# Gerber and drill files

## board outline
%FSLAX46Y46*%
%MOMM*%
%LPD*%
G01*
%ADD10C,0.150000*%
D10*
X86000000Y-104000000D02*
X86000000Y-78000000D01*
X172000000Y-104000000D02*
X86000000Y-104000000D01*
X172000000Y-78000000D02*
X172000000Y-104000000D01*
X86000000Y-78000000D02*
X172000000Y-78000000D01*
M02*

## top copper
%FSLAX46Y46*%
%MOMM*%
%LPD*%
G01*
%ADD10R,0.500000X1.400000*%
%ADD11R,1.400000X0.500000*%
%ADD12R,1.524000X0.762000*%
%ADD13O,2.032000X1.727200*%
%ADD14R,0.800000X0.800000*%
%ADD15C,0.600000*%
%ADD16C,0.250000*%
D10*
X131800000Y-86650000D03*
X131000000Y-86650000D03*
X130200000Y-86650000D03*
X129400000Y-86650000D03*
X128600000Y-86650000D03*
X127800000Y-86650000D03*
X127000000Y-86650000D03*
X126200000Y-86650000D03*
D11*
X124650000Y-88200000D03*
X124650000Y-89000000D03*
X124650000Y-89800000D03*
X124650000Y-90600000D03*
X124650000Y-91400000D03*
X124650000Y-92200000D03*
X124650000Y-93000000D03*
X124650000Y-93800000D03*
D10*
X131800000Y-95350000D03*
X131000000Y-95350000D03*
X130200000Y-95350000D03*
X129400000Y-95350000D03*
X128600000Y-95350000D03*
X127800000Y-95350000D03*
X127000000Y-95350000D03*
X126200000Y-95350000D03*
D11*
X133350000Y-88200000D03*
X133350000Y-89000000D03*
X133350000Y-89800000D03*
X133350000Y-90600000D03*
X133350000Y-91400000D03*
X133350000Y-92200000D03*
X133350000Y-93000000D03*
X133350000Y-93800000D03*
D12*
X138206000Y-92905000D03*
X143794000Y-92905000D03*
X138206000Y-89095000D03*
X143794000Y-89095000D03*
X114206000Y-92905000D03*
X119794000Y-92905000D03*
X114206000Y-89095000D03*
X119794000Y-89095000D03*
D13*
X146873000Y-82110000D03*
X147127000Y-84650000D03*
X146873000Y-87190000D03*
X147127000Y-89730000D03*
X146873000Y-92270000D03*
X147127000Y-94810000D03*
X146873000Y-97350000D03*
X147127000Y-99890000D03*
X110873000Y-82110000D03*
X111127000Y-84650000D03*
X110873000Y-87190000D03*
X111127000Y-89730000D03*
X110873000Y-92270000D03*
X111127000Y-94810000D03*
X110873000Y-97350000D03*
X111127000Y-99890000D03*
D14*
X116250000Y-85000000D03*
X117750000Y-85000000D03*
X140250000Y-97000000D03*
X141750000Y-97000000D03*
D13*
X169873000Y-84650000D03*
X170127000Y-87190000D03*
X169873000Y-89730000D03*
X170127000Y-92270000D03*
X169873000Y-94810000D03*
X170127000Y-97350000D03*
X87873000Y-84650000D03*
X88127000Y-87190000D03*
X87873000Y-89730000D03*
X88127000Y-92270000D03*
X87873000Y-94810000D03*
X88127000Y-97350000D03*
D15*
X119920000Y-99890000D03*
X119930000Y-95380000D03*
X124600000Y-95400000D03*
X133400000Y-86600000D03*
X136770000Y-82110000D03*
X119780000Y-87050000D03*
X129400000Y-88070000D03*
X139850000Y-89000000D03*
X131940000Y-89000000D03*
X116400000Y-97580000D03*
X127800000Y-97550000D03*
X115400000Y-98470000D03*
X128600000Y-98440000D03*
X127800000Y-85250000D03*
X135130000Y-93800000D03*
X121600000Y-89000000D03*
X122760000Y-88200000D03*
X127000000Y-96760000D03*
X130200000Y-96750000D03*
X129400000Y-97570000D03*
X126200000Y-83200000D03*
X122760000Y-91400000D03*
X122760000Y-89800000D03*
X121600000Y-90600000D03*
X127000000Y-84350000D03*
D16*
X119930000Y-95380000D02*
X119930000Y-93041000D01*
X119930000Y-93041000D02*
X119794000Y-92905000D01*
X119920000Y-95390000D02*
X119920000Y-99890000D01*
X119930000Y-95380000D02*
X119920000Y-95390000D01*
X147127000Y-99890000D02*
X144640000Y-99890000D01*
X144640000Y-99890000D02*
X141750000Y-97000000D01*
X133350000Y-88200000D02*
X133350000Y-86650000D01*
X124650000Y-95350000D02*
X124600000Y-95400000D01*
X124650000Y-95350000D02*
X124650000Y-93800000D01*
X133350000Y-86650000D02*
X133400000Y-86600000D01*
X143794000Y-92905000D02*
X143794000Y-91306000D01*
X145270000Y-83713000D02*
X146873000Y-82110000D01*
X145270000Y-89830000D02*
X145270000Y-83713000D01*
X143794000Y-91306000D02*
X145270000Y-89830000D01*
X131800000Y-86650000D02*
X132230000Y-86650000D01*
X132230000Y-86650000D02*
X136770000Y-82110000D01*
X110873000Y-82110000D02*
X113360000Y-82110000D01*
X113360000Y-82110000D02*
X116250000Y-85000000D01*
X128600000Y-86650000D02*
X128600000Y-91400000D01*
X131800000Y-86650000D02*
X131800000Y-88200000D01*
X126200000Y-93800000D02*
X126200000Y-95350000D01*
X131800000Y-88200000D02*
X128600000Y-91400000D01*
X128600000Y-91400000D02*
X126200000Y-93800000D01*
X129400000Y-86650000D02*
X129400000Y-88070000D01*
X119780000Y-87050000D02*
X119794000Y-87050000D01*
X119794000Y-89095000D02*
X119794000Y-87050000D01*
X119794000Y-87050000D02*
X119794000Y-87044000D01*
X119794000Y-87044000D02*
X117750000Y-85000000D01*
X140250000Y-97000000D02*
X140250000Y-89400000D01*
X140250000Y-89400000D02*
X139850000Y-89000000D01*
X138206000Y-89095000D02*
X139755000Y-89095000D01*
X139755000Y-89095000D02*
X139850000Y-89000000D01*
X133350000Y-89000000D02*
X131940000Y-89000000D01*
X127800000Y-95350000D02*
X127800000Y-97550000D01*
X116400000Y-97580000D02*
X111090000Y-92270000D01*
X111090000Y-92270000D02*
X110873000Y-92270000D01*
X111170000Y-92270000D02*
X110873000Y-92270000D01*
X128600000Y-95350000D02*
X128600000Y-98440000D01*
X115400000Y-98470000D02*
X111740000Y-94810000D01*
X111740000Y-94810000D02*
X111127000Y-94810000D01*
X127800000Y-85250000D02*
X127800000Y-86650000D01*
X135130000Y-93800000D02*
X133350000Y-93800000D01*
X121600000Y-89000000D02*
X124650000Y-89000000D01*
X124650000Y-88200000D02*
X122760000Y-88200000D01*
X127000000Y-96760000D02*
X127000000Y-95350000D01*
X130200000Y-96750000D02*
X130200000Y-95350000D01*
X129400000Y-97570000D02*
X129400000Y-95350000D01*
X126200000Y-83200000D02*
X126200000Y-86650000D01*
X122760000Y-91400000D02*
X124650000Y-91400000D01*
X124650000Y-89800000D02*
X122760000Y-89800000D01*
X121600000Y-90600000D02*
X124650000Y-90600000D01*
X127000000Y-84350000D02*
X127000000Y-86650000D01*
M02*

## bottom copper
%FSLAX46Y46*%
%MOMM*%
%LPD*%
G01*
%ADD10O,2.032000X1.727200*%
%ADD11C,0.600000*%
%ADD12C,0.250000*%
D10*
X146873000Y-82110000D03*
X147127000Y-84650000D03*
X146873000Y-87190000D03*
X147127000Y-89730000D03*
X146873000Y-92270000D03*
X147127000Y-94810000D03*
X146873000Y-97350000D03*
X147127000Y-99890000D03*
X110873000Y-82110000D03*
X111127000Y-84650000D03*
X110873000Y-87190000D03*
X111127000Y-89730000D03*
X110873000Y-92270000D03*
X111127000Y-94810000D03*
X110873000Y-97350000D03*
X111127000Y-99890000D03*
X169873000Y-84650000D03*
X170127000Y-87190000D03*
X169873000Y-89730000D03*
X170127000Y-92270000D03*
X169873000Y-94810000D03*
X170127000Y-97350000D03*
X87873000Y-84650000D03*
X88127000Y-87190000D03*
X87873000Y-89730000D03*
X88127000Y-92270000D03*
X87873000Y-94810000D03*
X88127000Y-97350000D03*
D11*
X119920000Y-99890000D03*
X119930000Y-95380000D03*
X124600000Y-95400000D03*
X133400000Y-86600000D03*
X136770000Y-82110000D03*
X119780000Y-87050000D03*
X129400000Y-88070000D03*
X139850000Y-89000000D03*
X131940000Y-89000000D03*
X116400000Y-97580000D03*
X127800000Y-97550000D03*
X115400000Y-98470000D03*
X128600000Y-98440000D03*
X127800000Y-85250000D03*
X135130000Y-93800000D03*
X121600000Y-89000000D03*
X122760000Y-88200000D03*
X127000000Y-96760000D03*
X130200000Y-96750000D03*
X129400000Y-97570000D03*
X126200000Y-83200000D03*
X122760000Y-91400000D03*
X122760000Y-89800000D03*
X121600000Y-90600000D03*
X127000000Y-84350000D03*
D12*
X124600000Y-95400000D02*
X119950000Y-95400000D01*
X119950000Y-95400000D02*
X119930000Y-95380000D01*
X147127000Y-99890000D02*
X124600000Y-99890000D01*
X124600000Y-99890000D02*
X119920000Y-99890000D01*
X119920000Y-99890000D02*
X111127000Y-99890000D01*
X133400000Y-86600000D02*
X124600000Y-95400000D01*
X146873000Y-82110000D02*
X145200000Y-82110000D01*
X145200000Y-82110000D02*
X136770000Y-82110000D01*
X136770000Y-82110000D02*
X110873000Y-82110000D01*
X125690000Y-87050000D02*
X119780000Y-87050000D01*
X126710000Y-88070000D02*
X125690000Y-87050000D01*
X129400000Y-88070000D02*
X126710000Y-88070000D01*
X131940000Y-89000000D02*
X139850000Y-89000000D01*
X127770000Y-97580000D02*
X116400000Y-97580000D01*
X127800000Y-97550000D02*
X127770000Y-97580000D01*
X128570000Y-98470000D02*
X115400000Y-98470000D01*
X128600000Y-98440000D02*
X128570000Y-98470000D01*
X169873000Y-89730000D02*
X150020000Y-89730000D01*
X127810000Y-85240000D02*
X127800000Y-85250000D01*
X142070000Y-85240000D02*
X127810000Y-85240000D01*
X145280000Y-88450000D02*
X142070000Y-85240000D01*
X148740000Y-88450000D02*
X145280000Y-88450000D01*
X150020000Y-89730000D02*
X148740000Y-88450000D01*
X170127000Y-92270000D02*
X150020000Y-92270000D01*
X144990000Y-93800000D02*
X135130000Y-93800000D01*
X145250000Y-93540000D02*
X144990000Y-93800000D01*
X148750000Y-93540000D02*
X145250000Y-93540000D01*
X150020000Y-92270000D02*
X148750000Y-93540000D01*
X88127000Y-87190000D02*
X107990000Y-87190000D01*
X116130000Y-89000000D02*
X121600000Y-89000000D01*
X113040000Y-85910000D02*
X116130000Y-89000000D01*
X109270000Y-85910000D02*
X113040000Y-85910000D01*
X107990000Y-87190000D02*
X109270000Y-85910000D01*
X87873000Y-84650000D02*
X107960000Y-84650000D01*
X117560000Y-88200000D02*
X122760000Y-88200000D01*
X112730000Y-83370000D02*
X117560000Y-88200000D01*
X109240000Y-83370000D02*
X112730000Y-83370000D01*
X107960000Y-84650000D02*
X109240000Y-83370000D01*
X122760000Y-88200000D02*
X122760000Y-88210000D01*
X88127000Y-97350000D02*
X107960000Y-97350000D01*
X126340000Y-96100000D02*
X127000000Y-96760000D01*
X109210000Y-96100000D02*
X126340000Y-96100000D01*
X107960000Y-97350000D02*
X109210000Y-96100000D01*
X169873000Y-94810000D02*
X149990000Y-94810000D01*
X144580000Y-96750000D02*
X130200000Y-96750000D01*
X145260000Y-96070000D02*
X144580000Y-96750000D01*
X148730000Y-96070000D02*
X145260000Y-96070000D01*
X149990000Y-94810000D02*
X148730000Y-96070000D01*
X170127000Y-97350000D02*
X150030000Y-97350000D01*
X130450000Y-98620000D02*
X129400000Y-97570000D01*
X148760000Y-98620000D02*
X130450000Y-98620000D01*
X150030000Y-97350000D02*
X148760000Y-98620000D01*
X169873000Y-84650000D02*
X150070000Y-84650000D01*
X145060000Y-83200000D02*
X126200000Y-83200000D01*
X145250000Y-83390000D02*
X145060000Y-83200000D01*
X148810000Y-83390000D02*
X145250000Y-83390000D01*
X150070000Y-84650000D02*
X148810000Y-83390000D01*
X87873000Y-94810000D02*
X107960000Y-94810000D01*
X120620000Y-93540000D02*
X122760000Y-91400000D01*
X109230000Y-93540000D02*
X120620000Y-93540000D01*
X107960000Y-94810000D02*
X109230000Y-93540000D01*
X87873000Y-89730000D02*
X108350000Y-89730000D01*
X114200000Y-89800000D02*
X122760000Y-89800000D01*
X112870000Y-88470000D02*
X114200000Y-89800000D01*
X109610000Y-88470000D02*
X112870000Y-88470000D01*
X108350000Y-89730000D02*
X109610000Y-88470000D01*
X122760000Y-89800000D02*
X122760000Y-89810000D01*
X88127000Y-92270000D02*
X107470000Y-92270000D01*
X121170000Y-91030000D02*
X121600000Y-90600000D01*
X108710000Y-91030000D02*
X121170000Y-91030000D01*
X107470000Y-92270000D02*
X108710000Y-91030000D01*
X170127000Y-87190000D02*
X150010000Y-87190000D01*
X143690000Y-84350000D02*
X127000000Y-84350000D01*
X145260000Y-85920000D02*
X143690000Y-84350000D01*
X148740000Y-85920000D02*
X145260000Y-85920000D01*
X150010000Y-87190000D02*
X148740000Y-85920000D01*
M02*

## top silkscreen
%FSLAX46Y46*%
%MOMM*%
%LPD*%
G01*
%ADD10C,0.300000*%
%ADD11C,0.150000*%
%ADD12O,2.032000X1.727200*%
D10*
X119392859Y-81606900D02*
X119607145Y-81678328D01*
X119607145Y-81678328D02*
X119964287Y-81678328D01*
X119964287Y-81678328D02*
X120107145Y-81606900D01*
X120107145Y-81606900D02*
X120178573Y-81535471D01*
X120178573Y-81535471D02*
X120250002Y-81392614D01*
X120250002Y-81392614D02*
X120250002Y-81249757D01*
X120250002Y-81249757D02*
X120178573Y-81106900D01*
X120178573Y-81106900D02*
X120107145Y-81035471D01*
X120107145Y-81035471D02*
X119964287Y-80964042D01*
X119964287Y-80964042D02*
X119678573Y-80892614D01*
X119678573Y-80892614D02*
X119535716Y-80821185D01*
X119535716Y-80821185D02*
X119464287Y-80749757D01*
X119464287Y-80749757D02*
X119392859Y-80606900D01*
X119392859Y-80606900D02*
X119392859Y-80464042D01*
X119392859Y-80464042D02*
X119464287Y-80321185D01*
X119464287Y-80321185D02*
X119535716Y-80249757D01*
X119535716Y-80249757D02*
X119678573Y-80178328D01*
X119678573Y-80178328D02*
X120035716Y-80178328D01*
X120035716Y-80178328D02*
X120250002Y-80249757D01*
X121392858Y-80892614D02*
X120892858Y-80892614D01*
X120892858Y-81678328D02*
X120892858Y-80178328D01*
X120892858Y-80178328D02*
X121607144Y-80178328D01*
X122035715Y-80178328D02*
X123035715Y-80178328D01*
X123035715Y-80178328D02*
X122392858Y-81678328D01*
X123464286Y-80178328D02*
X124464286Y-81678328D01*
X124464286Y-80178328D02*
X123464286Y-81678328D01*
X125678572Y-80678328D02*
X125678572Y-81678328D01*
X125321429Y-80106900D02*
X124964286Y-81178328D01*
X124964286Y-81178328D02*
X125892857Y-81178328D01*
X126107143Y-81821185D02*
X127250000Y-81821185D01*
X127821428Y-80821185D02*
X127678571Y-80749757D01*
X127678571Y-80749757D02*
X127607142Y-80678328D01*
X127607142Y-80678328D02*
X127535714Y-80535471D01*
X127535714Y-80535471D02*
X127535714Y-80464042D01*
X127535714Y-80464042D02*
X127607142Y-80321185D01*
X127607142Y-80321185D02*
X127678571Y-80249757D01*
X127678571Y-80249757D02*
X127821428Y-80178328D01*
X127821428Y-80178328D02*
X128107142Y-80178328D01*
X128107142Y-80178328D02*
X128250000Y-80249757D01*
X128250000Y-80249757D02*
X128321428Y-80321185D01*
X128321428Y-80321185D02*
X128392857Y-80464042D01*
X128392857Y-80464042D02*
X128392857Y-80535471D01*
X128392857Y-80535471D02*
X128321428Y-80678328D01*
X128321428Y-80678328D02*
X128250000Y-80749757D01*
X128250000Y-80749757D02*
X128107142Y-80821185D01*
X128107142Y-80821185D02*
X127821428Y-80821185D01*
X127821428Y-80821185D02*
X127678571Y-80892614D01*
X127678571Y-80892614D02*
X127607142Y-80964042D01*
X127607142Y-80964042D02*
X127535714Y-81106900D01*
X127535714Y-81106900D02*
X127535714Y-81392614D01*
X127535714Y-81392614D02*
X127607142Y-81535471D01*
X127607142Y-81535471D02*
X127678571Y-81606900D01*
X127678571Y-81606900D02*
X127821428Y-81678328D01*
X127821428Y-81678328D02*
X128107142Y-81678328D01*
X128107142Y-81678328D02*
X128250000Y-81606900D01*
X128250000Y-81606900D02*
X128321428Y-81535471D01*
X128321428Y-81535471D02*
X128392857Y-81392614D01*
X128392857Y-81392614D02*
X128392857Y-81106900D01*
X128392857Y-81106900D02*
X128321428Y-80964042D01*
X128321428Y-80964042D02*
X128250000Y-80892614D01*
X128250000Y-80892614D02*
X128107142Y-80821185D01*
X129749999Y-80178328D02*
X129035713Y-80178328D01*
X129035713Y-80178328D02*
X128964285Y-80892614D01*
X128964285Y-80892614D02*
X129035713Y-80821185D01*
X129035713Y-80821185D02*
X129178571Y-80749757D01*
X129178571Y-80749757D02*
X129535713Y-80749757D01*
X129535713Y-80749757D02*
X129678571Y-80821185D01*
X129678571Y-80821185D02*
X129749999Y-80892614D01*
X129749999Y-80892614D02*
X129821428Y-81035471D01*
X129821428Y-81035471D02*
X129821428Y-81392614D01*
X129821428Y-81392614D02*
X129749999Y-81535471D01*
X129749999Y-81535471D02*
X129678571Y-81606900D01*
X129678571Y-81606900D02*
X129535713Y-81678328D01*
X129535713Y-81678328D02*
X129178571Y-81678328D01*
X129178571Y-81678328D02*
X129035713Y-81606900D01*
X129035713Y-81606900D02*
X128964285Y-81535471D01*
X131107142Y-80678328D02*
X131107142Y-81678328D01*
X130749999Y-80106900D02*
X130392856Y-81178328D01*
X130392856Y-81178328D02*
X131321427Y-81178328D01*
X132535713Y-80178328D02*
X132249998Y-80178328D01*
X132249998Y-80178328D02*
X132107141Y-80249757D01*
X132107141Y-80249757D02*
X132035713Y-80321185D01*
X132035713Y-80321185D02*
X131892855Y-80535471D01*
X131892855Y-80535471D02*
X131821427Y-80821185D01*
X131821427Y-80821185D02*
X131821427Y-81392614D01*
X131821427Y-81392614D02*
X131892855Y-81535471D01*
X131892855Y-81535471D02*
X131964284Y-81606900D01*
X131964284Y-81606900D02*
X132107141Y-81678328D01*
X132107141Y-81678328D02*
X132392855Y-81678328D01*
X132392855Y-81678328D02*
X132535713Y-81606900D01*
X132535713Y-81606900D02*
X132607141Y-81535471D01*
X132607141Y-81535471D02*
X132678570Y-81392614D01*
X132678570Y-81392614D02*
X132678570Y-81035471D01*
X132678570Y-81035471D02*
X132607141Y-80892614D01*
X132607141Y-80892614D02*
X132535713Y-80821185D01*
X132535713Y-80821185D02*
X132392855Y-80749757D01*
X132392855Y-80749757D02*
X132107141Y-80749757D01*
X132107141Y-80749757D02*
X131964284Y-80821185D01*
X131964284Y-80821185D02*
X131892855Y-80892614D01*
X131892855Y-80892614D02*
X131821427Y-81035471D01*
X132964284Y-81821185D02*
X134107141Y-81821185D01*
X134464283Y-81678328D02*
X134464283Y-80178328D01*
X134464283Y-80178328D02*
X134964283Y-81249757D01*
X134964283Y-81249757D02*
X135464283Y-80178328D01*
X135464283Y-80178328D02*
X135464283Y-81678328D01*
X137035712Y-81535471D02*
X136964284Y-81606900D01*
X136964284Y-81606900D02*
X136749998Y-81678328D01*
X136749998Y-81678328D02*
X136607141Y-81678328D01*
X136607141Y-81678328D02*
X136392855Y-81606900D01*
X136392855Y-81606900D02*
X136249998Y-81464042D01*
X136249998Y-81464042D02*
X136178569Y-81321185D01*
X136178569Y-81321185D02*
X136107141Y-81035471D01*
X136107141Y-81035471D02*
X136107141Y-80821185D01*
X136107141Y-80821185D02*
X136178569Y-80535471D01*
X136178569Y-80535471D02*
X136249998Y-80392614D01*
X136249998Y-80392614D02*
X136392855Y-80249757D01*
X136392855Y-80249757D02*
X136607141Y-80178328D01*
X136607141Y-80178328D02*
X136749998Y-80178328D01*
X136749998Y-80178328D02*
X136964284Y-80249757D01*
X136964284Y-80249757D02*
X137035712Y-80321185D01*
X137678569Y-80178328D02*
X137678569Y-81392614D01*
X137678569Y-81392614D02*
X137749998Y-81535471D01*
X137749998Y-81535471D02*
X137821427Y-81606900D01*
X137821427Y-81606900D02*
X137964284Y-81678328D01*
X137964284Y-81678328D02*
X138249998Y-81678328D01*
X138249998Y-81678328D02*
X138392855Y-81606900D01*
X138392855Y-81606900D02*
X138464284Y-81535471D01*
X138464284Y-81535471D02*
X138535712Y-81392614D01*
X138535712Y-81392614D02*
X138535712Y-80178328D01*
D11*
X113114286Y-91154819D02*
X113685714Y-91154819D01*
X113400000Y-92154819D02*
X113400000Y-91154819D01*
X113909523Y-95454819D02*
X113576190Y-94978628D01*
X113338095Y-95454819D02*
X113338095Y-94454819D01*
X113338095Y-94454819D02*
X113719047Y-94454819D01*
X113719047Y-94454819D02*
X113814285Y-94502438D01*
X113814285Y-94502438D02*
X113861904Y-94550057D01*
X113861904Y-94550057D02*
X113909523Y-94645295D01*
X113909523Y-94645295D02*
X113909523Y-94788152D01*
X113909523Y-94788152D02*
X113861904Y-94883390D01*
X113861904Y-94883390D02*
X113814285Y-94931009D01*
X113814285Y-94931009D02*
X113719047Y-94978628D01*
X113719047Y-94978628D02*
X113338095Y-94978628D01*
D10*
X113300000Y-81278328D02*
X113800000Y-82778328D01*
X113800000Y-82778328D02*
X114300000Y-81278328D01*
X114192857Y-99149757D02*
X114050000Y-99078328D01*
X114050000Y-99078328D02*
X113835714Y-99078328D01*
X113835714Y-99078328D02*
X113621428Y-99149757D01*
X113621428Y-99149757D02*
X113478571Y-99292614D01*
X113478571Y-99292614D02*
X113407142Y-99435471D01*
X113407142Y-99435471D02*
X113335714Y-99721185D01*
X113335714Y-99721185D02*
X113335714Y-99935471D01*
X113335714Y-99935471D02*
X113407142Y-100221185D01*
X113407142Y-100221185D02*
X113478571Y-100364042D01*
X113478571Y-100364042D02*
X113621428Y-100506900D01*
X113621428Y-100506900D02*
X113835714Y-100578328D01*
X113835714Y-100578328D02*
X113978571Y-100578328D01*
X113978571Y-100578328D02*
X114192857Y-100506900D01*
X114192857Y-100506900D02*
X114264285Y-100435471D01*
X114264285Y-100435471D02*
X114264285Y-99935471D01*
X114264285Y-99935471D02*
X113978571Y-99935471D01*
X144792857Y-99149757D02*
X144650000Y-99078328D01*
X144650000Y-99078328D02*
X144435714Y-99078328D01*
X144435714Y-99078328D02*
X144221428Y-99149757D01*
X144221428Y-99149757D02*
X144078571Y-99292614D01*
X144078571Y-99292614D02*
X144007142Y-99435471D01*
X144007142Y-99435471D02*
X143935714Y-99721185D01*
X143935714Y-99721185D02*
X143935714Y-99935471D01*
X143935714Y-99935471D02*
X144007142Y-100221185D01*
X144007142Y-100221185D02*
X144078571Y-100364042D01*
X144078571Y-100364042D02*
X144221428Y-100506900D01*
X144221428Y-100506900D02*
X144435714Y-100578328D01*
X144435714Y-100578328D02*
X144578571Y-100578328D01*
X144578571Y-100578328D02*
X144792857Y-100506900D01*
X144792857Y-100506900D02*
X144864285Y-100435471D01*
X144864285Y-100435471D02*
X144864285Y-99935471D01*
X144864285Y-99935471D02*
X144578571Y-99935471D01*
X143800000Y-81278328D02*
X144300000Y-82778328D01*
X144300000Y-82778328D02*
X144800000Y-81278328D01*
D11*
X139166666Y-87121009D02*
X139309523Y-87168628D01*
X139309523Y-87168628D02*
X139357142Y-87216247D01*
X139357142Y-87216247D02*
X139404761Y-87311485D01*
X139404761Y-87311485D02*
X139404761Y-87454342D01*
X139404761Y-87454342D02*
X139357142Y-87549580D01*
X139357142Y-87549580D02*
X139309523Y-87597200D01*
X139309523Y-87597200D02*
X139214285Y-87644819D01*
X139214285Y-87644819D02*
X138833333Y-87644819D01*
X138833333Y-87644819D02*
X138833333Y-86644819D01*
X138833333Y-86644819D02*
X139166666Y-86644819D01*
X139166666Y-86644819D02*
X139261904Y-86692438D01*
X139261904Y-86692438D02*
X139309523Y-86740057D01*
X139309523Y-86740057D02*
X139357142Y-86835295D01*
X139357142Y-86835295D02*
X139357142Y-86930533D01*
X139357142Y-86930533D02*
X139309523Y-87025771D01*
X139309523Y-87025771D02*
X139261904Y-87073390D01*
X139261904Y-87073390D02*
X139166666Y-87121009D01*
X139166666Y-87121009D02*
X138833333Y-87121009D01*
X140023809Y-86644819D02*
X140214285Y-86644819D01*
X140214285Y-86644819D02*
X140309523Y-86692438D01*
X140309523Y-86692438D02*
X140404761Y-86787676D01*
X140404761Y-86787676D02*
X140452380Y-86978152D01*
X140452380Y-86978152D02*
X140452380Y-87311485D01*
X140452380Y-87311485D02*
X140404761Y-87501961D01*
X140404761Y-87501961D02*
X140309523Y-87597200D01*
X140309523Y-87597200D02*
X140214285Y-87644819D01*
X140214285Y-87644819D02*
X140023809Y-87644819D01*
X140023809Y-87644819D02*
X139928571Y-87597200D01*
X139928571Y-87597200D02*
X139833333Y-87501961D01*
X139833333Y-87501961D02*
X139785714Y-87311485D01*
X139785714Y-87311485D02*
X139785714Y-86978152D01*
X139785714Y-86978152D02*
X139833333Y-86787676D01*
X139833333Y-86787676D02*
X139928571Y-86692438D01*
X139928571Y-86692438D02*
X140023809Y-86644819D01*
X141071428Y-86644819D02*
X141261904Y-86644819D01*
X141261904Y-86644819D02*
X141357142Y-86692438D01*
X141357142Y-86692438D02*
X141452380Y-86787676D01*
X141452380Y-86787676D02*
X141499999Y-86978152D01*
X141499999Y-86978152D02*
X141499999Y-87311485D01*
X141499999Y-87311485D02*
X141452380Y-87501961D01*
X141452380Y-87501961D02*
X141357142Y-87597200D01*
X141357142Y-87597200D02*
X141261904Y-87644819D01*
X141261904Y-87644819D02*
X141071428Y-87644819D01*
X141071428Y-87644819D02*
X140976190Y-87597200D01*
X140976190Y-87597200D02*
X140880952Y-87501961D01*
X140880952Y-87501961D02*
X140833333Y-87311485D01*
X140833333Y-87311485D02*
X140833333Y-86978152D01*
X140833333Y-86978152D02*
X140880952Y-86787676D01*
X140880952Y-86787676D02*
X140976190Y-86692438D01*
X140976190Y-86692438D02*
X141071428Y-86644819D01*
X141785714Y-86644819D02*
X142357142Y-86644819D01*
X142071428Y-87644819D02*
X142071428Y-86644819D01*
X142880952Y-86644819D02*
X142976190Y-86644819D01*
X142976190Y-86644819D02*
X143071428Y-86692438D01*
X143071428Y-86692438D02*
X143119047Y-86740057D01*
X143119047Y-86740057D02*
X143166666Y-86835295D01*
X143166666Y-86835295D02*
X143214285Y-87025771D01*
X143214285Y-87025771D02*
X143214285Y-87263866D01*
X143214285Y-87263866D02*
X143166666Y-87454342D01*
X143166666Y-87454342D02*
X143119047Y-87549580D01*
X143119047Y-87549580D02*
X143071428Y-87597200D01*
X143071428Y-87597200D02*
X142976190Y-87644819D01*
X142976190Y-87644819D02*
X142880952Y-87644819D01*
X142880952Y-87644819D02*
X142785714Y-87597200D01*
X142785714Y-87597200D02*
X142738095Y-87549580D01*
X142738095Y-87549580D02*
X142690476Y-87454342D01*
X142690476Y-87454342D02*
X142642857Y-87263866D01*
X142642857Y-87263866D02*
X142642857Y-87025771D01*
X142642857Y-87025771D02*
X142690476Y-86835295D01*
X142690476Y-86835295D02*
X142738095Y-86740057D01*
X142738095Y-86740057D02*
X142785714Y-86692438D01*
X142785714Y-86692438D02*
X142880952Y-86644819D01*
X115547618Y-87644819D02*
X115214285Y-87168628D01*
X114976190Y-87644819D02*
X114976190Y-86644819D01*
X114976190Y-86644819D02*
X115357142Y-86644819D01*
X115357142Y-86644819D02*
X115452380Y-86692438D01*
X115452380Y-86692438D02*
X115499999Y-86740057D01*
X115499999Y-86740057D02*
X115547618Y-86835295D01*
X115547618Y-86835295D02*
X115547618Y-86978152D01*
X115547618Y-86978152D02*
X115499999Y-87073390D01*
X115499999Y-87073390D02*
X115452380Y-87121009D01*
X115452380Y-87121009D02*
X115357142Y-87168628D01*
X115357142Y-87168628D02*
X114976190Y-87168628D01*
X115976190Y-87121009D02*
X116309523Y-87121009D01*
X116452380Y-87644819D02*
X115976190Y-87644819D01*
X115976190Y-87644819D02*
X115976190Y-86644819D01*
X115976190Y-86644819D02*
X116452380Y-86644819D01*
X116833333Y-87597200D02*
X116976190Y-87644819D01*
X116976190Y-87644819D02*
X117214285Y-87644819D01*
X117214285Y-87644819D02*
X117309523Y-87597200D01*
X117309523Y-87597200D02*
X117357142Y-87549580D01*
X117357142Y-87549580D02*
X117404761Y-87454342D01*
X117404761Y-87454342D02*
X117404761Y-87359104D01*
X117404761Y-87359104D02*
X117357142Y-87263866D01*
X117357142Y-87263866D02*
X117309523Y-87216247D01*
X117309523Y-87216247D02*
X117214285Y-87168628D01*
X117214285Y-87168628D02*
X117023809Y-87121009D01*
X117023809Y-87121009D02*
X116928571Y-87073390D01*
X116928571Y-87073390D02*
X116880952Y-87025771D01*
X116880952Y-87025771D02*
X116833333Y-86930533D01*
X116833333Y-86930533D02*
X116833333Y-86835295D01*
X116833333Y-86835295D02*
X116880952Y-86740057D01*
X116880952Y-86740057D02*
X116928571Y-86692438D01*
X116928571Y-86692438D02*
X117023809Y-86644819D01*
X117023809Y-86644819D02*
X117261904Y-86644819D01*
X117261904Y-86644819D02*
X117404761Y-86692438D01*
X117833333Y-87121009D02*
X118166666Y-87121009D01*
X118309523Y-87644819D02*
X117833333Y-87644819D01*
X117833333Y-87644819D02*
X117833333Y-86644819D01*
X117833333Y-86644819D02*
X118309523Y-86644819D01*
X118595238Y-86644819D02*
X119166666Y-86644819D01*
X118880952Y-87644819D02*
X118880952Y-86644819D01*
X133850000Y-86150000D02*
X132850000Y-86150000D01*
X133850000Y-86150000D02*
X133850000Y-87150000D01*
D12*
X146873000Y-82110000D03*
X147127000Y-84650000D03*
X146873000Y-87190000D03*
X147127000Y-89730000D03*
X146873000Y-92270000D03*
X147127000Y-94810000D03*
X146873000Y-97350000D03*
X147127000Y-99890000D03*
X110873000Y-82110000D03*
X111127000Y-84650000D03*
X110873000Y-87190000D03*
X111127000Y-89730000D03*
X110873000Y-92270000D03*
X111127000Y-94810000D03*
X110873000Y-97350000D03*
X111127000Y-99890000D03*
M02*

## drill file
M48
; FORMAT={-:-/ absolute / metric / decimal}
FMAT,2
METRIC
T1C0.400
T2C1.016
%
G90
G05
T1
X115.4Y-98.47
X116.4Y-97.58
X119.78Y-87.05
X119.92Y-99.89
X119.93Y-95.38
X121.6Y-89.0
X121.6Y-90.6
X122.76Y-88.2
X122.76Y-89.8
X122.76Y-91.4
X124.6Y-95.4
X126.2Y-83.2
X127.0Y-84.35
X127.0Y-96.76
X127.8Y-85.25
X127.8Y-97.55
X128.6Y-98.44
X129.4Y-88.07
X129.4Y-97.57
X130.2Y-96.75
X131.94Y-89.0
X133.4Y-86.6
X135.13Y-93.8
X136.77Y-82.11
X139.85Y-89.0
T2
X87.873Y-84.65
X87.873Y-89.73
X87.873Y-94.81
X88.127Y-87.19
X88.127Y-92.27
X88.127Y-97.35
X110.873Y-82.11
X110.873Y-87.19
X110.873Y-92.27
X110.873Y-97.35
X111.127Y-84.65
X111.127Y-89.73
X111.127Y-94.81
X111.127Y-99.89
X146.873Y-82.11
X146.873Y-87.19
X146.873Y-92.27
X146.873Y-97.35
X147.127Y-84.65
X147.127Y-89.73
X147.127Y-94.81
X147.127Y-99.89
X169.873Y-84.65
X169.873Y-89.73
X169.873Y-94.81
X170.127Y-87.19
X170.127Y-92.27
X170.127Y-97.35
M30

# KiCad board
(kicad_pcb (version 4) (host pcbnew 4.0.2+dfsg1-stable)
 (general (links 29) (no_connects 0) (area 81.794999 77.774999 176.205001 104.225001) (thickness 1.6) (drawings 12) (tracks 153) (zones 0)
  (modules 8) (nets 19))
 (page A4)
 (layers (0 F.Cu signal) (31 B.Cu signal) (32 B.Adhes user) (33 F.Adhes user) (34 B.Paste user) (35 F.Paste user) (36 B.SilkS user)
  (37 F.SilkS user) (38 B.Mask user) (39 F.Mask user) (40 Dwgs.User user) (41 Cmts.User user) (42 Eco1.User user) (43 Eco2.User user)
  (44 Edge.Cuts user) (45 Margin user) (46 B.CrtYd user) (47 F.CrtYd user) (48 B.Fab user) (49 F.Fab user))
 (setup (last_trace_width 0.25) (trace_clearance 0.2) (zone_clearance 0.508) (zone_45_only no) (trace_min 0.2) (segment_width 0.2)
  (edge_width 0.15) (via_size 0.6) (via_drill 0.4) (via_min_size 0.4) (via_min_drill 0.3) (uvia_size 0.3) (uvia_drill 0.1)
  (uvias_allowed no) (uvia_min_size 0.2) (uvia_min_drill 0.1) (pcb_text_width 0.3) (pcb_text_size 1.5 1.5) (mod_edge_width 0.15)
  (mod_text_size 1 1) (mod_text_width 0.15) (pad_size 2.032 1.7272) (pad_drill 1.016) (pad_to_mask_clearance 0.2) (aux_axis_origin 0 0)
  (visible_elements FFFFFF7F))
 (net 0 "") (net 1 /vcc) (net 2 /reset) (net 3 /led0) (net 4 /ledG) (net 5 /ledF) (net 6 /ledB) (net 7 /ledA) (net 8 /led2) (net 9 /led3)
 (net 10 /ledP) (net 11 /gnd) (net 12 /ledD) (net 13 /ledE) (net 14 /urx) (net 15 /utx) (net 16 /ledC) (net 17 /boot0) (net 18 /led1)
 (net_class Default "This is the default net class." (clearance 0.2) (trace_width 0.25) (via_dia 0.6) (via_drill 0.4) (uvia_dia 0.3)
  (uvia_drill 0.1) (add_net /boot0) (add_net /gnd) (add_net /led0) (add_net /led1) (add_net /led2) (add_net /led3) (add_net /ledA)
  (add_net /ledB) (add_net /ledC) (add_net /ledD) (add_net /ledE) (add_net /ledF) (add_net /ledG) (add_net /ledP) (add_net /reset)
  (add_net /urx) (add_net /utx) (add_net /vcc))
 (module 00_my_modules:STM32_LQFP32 (layer F.Cu) (at 129 91 270)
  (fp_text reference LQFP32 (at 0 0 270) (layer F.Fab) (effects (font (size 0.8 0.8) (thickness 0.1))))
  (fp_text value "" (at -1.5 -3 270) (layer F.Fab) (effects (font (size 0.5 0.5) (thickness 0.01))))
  (fp_line (start -4.85 -4.85) (end -4.85 -3.85) (layer F.SilkS) (width 0.15))
  (fp_line (start -4.85 -4.85) (end -3.85 -4.85) (layer F.SilkS) (width 0.15))
  (pad 3.3 smd rect (at -4.35 -2.8 270) (size 1.4 0.5) (layers F.Cu F.Paste F.Mask) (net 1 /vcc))
  (pad PF0 smd rect (at -4.35 -2 270) (size 1.4 0.5) (layers F.Cu F.Paste F.Mask))
  (pad PF1 smd rect (at -4.35 -1.2 270) (size 1.4 0.5) (layers F.Cu F.Paste F.Mask))
  (pad RST smd rect (at -4.35 -0.4 270) (size 1.4 0.5) (layers F.Cu F.Paste F.Mask) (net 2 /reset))
  (pad 3.3 smd rect (at -4.35 0.4 270) (size 1.4 0.5) (layers F.Cu F.Paste F.Mask) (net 1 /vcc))
  (pad PA0 smd rect (at -4.35 1.2 270) (size 1.4 0.5) (layers F.Cu F.Paste F.Mask) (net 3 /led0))
  (pad PA1 smd rect (at -4.35 2 270) (size 1.4 0.5) (layers F.Cu F.Paste F.Mask) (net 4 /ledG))
  (pad PA2 smd rect (at -4.35 2.8 270) (size 1.4 0.5) (layers F.Cu F.Paste F.Mask) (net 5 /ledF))
  (pad PA3 smd rect (at -2.8 4.35) (size 1.4 0.5) (layers F.Cu F.Paste F.Mask) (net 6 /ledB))
  (pad PA4 smd rect (at -2 4.35) (size 1.4 0.5) (layers F.Cu F.Paste F.Mask) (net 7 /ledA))
  (pad PA5 smd rect (at -1.2 4.35) (size 1.4 0.5) (layers F.Cu F.Paste F.Mask) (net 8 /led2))
  (pad PA6 smd rect (at -0.4 4.35) (size 1.4 0.5) (layers F.Cu F.Paste F.Mask) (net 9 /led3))
  (pad PA7 smd rect (at 0.4 4.35) (size 1.4 0.5) (layers F.Cu F.Paste F.Mask) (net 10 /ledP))
  (pad PB0 smd rect (at 1.2 4.35) (size 1.4 0.5) (layers F.Cu F.Paste F.Mask))
  (pad PB1 smd rect (at 2 4.35) (size 1.4 0.5) (layers F.Cu F.Paste F.Mask))
  (pad GND smd rect (at 2.8 4.35) (size 1.4 0.5) (layers F.Cu F.Paste F.Mask) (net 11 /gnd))
  (pad PA14 smd rect (at 4.35 -2.8 270) (size 1.4 0.5) (layers F.Cu F.Paste F.Mask))
  (pad PA13 smd rect (at 4.35 -2 270) (size 1.4 0.5) (layers F.Cu F.Paste F.Mask))
  (pad PA12 smd rect (at 4.35 -1.2 270) (size 1.4 0.5) (layers F.Cu F.Paste F.Mask) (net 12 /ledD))
  (pad PA11 smd rect (at 4.35 -0.4 270) (size 1.4 0.5) (layers F.Cu F.Paste F.Mask) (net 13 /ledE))
  (pad PA10 smd rect (at 4.35 0.4 270) (size 1.4 0.5) (layers F.Cu F.Paste F.Mask) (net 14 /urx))
  (pad PA9 smd rect (at 4.35 1.2 270) (size 1.4 0.5) (layers F.Cu F.Paste F.Mask) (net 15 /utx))
  (pad PA8 smd rect (at 4.35 2 270) (size 1.4 0.5) (layers F.Cu F.Paste F.Mask) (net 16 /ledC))
  (pad 3.3 smd rect (at 4.35 2.8 270) (size 1.4 0.5) (layers F.Cu F.Paste F.Mask) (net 1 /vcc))
  (pad GND smd rect (at -2.8 -4.35) (size 1.4 0.5) (layers F.Cu F.Paste F.Mask) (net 11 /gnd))
  (pad BOOT smd rect (at -2 -4.35) (size 1.4 0.5) (layers F.Cu F.Paste F.Mask) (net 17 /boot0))
  (pad PB7 smd rect (at -1.2 -4.35) (size 1.4 0.5) (layers F.Cu F.Paste F.Mask))
  (pad PB6 smd rect (at -0.4 -4.35) (size 1.4 0.5) (layers F.Cu F.Paste F.Mask))
  (pad PB5 smd rect (at 0.4 -4.35) (size 1.4 0.5) (layers F.Cu F.Paste F.Mask))
  (pad PB4 smd rect (at 1.2 -4.35) (size 1.4 0.5) (layers F.Cu F.Paste F.Mask))
  (pad PB3 smd rect (at 2 -4.35) (size 1.4 0.5) (layers F.Cu F.Paste F.Mask))
  (pad PA15 smd rect (at 2.8 -4.35) (size 1.4 0.5) (layers F.Cu F.Paste F.Mask) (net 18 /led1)))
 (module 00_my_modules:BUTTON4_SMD (layer F.Cu) (at 141 91)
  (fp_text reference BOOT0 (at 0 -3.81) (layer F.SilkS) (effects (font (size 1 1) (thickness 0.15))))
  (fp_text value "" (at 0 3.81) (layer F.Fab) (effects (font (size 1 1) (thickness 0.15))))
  (pad 1 smd rect (at -2.794 1.905) (size 1.524 0.762) (layers F.Cu F.Paste F.Mask))
  (pad 2 smd rect (at 2.794 1.905) (size 1.524 0.762) (layers F.Cu F.Paste F.Mask) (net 1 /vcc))
  (pad 3 smd rect (at -2.794 -1.905) (size 1.524 0.762) (layers F.Cu F.Paste F.Mask) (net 17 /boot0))
  (pad 4 smd rect (at 2.794 -1.905) (size 1.524 0.762) (layers F.Cu F.Paste F.Mask)))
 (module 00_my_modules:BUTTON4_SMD (layer F.Cu) (at 117 91)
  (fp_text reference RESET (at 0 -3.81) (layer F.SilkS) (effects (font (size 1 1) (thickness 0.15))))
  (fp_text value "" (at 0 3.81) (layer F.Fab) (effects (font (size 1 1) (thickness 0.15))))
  (pad 1 smd rect (at -2.794 1.905) (size 1.524 0.762) (layers F.Cu F.Paste F.Mask))
  (pad 2 smd rect (at 2.794 1.905) (size 1.524 0.762) (layers F.Cu F.Paste F.Mask) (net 11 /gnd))
  (pad 3 smd rect (at -2.794 -1.905) (size 1.524 0.762) (layers F.Cu F.Paste F.Mask))
  (pad 4 smd rect (at 2.794 -1.905) (size 1.524 0.762) (layers F.Cu F.Paste F.Mask) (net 2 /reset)))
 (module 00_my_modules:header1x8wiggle (layer F.Cu) (at 147 91)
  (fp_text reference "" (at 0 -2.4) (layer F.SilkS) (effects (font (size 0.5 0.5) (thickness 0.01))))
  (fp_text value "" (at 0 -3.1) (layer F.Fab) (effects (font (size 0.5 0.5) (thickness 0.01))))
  (pad 1 thru_hole oval (at -0.127 -8.89) (size 2.032 1.7272) (drill 1.016) (layers *.Cu *.Mask F.SilkS) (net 1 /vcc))
  (pad 2 thru_hole oval (at 0.127 -6.35) (size 2.032 1.7272) (drill 1.016) (layers *.Cu *.Mask F.SilkS))
  (pad 3 thru_hole oval (at -0.127 -3.81) (size 2.032 1.7272) (drill 1.016) (layers *.Cu *.Mask F.SilkS))
  (pad 4 thru_hole oval (at 0.127 -1.27) (size 2.032 1.7272) (drill 1.016) (layers *.Cu *.Mask F.SilkS))
  (pad 5 thru_hole oval (at -0.127 1.27) (size 2.032 1.7272) (drill 1.016) (layers *.Cu *.Mask F.SilkS))
  (pad 6 thru_hole oval (at 0.127 3.81) (size 2.032 1.7272) (drill 1.016) (layers *.Cu *.Mask F.SilkS))
  (pad 7 thru_hole oval (at -0.127 6.35) (size 2.032 1.7272) (drill 1.016) (layers *.Cu *.Mask F.SilkS))
  (pad 8 thru_hole oval (at 0.127 8.89) (size 2.032 1.7272) (drill 1.016) (layers *.Cu *.Mask F.SilkS) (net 11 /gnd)))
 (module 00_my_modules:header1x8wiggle (layer F.Cu) (at 111 91)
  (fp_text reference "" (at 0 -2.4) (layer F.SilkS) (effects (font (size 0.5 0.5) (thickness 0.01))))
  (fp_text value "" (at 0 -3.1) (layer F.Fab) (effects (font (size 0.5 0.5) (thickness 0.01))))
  (pad 1 thru_hole oval (at -0.127 -8.89) (size 2.032 1.7272) (drill 1.016) (layers *.Cu *.Mask F.SilkS) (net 1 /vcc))
  (pad 2 thru_hole oval (at 0.127 -6.35) (size 2.032 1.7272) (drill 1.016) (layers *.Cu *.Mask F.SilkS))
  (pad 3 thru_hole oval (at -0.127 -3.81) (size 2.032 1.7272) (drill 1.016) (layers *.Cu *.Mask F.SilkS))
  (pad 4 thru_hole oval (at 0.127 -1.27) (size 2.032 1.7272) (drill 1.016) (layers *.Cu *.Mask F.SilkS))
  (pad 5 thru_hole oval (at -0.127 1.27) (size 2.032 1.7272) (drill 1.016) (layers *.Cu *.Mask F.SilkS) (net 15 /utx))
  (pad 6 thru_hole oval (at 0.127 3.81) (size 2.032 1.7272) (drill 1.016) (layers *.Cu *.Mask F.SilkS) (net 14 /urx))
  (pad 7 thru_hole oval (at -0.127 6.35) (size 2.032 1.7272) (drill 1.016) (layers *.Cu *.Mask F.SilkS))
  (pad 8 thru_hole oval (at 0.127 8.89) (size 2.032 1.7272) (drill 1.016) (layers *.Cu *.Mask F.SilkS) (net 11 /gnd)))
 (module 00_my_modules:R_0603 (layer F.Cu) (at 117 85)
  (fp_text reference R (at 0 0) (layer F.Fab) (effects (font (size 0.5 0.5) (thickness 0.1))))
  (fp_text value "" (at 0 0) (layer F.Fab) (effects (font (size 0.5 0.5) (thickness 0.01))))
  (pad 1 smd rect (at -0.75 0) (size 0.8 0.8) (layers F.Cu F.Paste F.Mask) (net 1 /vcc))
  (pad 2 smd rect (at 0.75 0) (size 0.8 0.8) (layers F.Cu F.Paste F.Mask) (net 2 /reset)))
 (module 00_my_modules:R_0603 (layer F.Cu) (at 141 97)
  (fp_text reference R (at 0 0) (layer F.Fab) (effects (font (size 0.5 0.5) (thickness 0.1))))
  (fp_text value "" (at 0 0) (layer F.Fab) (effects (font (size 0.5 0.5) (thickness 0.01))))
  (pad 1 smd rect (at -0.75 0) (size 0.8 0.8) (layers F.Cu F.Paste F.Mask) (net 17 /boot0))
  (pad 2 smd rect (at 0.75 0) (size 0.8 0.8) (layers F.Cu F.Paste F.Mask) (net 11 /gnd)))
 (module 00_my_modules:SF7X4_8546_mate (layer B.Cu) (at 129 91 180)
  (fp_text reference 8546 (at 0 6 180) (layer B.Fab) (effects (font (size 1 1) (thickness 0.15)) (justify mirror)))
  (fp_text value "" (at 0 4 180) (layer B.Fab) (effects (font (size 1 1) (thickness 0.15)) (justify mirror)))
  (pad F thru_hole oval (at -40.873 6.35 180) (size 2.032 1.7272) (drill 1.016) (layers *.Cu *.Mask B.SilkS) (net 5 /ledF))
  (pad G thru_hole oval (at -41.127 3.81 180) (size 2.032 1.7272) (drill 1.016) (layers *.Cu *.Mask B.SilkS) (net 4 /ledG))
  (pad V0 thru_hole oval (at -40.873 1.27 180) (size 2.032 1.7272) (drill 1.016) (layers *.Cu *.Mask B.SilkS) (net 3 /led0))
  (pad V1 thru_hole oval (at -41.127 -1.27 180) (size 2.032 1.7272) (drill 1.016) (layers *.Cu *.Mask B.SilkS) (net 18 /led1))
  (pad D thru_hole oval (at -40.873 -3.81 180) (size 2.032 1.7272) (drill 1.016) (layers *.Cu *.Mask B.SilkS) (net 12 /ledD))
  (pad E thru_hole oval (at -41.127 -6.35 180) (size 2.032 1.7272) (drill 1.016) (layers *.Cu *.Mask B.SilkS) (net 13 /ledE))
  (pad B thru_hole oval (at 41.127 6.35 180) (size 2.032 1.7272) (drill 1.016) (layers *.Cu *.Mask B.SilkS) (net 6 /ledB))
  (pad A thru_hole oval (at 40.873 3.81 180) (size 2.032 1.7272) (drill 1.016) (layers *.Cu *.Mask B.SilkS) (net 7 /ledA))
  (pad V2 thru_hole oval (at 41.127 1.27 180) (size 2.032 1.7272) (drill 1.016) (layers *.Cu *.Mask B.SilkS) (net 8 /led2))
  (pad V3 thru_hole oval (at 40.873 -1.27 180) (size 2.032 1.7272) (drill 1.016) (layers *.Cu *.Mask B.SilkS) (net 9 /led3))
  (pad P thru_hole oval (at 41.127 -3.81 180) (size 2.032 1.7272) (drill 1.016) (layers *.Cu *.Mask B.SilkS) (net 10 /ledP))
  (pad C thru_hole oval (at 40.873 -6.35 180) (size 2.032 1.7272) (drill 1.016) (layers *.Cu *.Mask B.SilkS) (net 16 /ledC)))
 (gr_line (start 86 104) (end 86 78) (angle 90) (layer Edge.Cuts) (width 0.15))
 (gr_line (start 172 104) (end 86 104) (angle 90) (layer Edge.Cuts) (width 0.15))
 (gr_line (start 172 78) (end 172 104) (angle 90) (layer Edge.Cuts) (width 0.15))
 (gr_line (start 86 78) (end 172 78) (angle 90) (layer Edge.Cuts) (width 0.15))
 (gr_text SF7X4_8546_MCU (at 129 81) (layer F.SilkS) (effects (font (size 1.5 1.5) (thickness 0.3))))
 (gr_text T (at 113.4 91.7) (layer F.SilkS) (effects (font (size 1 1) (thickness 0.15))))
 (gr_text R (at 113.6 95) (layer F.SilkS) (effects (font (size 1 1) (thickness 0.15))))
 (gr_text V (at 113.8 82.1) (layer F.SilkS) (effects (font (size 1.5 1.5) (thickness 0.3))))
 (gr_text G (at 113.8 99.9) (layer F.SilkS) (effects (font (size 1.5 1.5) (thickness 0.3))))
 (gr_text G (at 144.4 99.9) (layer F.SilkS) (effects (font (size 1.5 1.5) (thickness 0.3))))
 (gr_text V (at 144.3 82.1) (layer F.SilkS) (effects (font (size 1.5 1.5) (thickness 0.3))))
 (segment (start 119.93 95.38) (end 119.93 93.041) (width 0.25) (layer F.Cu) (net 11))
 (segment (start 119.93 93.041) (end 119.794 92.905) (width 0.25) (layer F.Cu) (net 11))
 (segment (start 124.6 95.4) (end 119.95 95.4) (width 0.25) (layer B.Cu) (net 11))
 (via (at 119.92 99.89) (size 0.6) (drill 0.4) (layers F.Cu B.Cu) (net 11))
 (segment (start 119.92 95.39) (end 119.92 99.89) (width 0.25) (layer F.Cu) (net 11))
 (segment (start 119.93 95.38) (end 119.92 95.39) (width 0.25) (layer F.Cu) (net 11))
 (via (at 119.93 95.38) (size 0.6) (drill 0.4) (layers F.Cu B.Cu) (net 11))
 (segment (start 119.95 95.4) (end 119.93 95.38) (width 0.25) (layer B.Cu) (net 11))
 (segment (start 147.127 99.89) (end 144.64 99.89) (width 0.25) (layer F.Cu) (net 11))
 (segment (start 144.64 99.89) (end 141.75 97) (width 0.25) (layer F.Cu) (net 11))
 (segment (start 147.127 99.89) (end 124.6 99.89) (width 0.25) (layer B.Cu) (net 11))
 (segment (start 124.6 99.89) (end 119.92 99.89) (width 0.25) (layer B.Cu) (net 11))
 (segment (start 119.92 99.89) (end 111.127 99.89) (width 0.25) (layer B.Cu) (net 11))
 (segment (start 133.35 88.2) (end 133.35 86.65) (width 0.25) (layer F.Cu) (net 11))
 (segment (start 124.65 95.35) (end 124.6 95.4) (width 0.25) (layer F.Cu) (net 11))
 (via (at 124.6 95.4) (size 0.6) (drill 0.4) (layers F.Cu B.Cu) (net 11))
 (segment (start 124.65 95.35) (end 124.65 93.8) (width 0.25) (layer F.Cu) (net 11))
 (segment (start 133.4 86.6) (end 124.6 95.4) (width 0.25) (layer B.Cu) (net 11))
 (via (at 133.4 86.6) (size 0.6) (drill 0.4) (layers F.Cu B.Cu) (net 11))
 (segment (start 133.35 86.65) (end 133.4 86.6) (width 0.25) (layer F.Cu) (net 11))
 (segment (start 143.794 92.905) (end 143.794 91.306) (width 0.25) (layer F.Cu) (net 1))
 (segment (start 145.27 83.713) (end 146.873 82.11) (width 0.25) (layer F.Cu) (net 1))
 (segment (start 145.27 89.83) (end 145.27 83.713) (width 0.25) (layer F.Cu) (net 1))
 (segment (start 143.794 91.306) (end 145.27 89.83) (width 0.25) (layer F.Cu) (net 1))
 (segment (start 131.8 86.65) (end 132.23 86.65) (width 0.25) (layer F.Cu) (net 1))
 (via (at 136.77 82.11) (size 0.6) (drill 0.4) (layers F.Cu B.Cu) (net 1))
 (segment (start 132.23 86.65) (end 136.77 82.11) (width 0.25) (layer F.Cu) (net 1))
 (segment (start 110.873 82.11) (end 113.36 82.11) (width 0.25) (layer F.Cu) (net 1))
 (segment (start 113.36 82.11) (end 116.25 85) (width 0.25) (layer F.Cu) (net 1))
 (segment (start 146.873 82.11) (end 145.2 82.11) (width 0.25) (layer B.Cu) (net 1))
 (segment (start 145.2 82.11) (end 136.77 82.11) (width 0.25) (layer B.Cu) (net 1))
 (segment (start 136.77 82.11) (end 110.873 82.11) (width 0.25) (layer B.Cu) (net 1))
 (segment (start 128.6 86.65) (end 128.6 91.4) (width 0.25) (layer F.Cu) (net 1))
 (segment (start 131.8 86.65) (end 131.8 88.2) (width 0.25) (layer F.Cu) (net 1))
 (segment (start 126.2 93.8) (end 126.2 95.35) (width 0.25) (layer F.Cu) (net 1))
 (segment (start 131.8 88.2) (end 128.6 91.4) (width 0.25) (layer F.Cu) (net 1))
 (segment (start 128.6 91.4) (end 126.2 93.8) (width 0.25) (layer F.Cu) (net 1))
 (segment (start 129.4 86.65) (end 129.4 88.07) (width 0.25) (layer F.Cu) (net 2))
 (segment (start 119.78 87.05) (end 119.794 87.05) (width 0.25) (layer F.Cu) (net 2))
 (via (at 119.78 87.05) (size 0.6) (drill 0.4) (layers F.Cu B.Cu) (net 2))
 (segment (start 125.69 87.05) (end 119.78 87.05) (width 0.25) (layer B.Cu) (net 2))
 (segment (start 126.71 88.07) (end 125.69 87.05) (width 0.25) (layer B.Cu) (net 2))
 (segment (start 129.4 88.07) (end 126.71 88.07) (width 0.25) (layer B.Cu) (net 2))
 (via (at 129.4 88.07) (size 0.6) (drill 0.4) (layers F.Cu B.Cu) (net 2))
 (segment (start 119.794 89.095) (end 119.794 87.05) (width 0.25) (layer F.Cu) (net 2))
 (segment (start 119.794 87.05) (end 119.794 87.044) (width 0.25) (layer F.Cu) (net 2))
 (segment (start 119.794 87.044) (end 117.75 85) (width 0.25) (layer F.Cu) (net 2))
 (segment (start 140.25 97) (end 140.25 89.4) (width 0.25) (layer F.Cu) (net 17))
 (segment (start 140.25 89.4) (end 139.85 89) (width 0.25) (layer F.Cu) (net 17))
 (via (at 139.85 89) (size 0.6) (drill 0.4) (layers F.Cu B.Cu) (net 17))
 (segment (start 138.206 89.095) (end 139.755 89.095) (width 0.25) (layer F.Cu) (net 17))
 (segment (start 139.755 89.095) (end 139.85 89) (width 0.25) (layer F.Cu) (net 17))
 (segment (start 133.35 89) (end 131.94 89) (width 0.25) (layer F.Cu) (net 17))
 (segment (start 131.94 89) (end 139.85 89) (width 0.25) (layer B.Cu) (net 17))
 (via (at 131.94 89) (size 0.6) (drill 0.4) (layers F.Cu B.Cu) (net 17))
 (segment (start 127.8 95.35) (end 127.8 97.55) (width 0.25) (layer F.Cu) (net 15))
 (segment (start 116.4 97.58) (end 111.09 92.27) (width 0.25) (layer F.Cu) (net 15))
 (via (at 116.4 97.58) (size 0.6) (drill 0.4) (layers F.Cu B.Cu) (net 15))
 (segment (start 127.77 97.58) (end 116.4 97.58) (width 0.25) (layer B.Cu) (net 15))
 (segment (start 127.8 97.55) (end 127.77 97.58) (width 0.25) (layer B.Cu) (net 15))
 (via (at 127.8 97.55) (size 0.6) (drill 0.4) (layers F.Cu B.Cu) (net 15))
 (segment (start 111.09 92.27) (end 110.873 92.27) (width 0.25) (layer F.Cu) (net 15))
 (segment (start 111.17 92.27) (end 110.873 92.27) (width 0.25) (layer F.Cu) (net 15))
 (segment (start 128.6 95.35) (end 128.6 98.44) (width 0.25) (layer F.Cu) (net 14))
 (segment (start 115.4 98.47) (end 111.74 94.81) (width 0.25) (layer F.Cu) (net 14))
 (via (at 115.4 98.47) (size 0.6) (drill 0.4) (layers F.Cu B.Cu) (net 14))
 (segment (start 128.57 98.47) (end 115.4 98.47) (width 0.25) (layer B.Cu) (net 14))
 (segment (start 128.6 98.44) (end 128.57 98.47) (width 0.25) (layer B.Cu) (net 14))
 (via (at 128.6 98.44) (size 0.6) (drill 0.4) (layers F.Cu B.Cu) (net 14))
 (segment (start 111.74 94.81) (end 111.127 94.81) (width 0.25) (layer F.Cu) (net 14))
 (segment (start 169.873 89.73) (end 150.02 89.73) (width 0.25) (layer B.Cu) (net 3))
 (via (at 127.8 85.25) (size 0.6) (drill 0.4) (layers F.Cu B.Cu) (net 3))
 (segment (start 127.8 85.25) (end 127.8 86.65) (width 0.25) (layer F.Cu) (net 3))
 (segment (start 127.81 85.24) (end 127.8 85.25) (width 0.25) (layer B.Cu) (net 3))
 (segment (start 142.07 85.24) (end 127.81 85.24) (width 0.25) (layer B.Cu) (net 3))
 (segment (start 145.28 88.45) (end 142.07 85.24) (width 0.25) (layer B.Cu) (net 3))
 (segment (start 148.74 88.45) (end 145.28 88.45) (width 0.25) (layer B.Cu) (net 3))
 (segment (start 150.02 89.73) (end 148.74 88.45) (width 0.25) (layer B.Cu) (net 3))
 (segment (start 170.127 92.27) (end 150.02 92.27) (width 0.25) (layer B.Cu) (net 18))
 (via (at 135.13 93.8) (size 0.6) (drill 0.4) (layers F.Cu B.Cu) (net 18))
 (segment (start 135.13 93.8) (end 133.35 93.8) (width 0.25) (layer F.Cu) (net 18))
 (segment (start 144.99 93.8) (end 135.13 93.8) (width 0.25) (layer B.Cu) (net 18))
 (segment (start 145.25 93.54) (end 144.99 93.8) (width 0.25) (layer B.Cu) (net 18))
 (segment (start 148.75 93.54) (end 145.25 93.54) (width 0.25) (layer B.Cu) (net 18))
 (segment (start 150.02 92.27) (end 148.75 93.54) (width 0.25) (layer B.Cu) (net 18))
 (segment (start 88.127 87.19) (end 107.99 87.19) (width 0.25) (layer B.Cu) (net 7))
 (via (at 121.6 89) (size 0.6) (drill 0.4) (layers F.Cu B.Cu) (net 7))
 (segment (start 121.6 89) (end 124.65 89) (width 0.25) (layer F.Cu) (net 7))
 (segment (start 116.13 89) (end 121.6 89) (width 0.25) (layer B.Cu) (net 7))
 (segment (start 113.04 85.91) (end 116.13 89) (width 0.25) (layer B.Cu) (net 7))
 (segment (start 109.27 85.91) (end 113.04 85.91) (width 0.25) (layer B.Cu) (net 7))
 (segment (start 107.99 87.19) (end 109.27 85.91) (width 0.25) (layer B.Cu) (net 7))
 (segment (start 87.873 84.65) (end 107.96 84.65) (width 0.25) (layer B.Cu) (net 6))
 (segment (start 117.56 88.2) (end 122.76 88.2) (width 0.25) (layer B.Cu) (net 6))
 (segment (start 112.73 83.37) (end 117.56 88.2) (width 0.25) (layer B.Cu) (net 6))
 (segment (start 109.24 83.37) (end 112.73 83.37) (width 0.25) (layer B.Cu) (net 6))
 (segment (start 107.96 84.65) (end 109.24 83.37) (width 0.25) (layer B.Cu) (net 6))
 (segment (start 124.65 88.2) (end 122.76 88.2) (width 0.25) (layer F.Cu) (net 6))
 (segment (start 122.76 88.2) (end 122.76 88.21) (width 0.25) (layer B.Cu) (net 6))
 (via (at 122.76 88.2) (size 0.6) (drill 0.4) (layers F.Cu B.Cu) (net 6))
 (segment (start 88.127 97.35) (end 107.96 97.35) (width 0.25) (layer B.Cu) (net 16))
 (segment (start 127 96.76) (end 127 95.35) (width 0.25) (layer F.Cu) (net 16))
 (via (at 127 96.76) (size 0.6) (drill 0.4) (layers F.Cu B.Cu) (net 16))
 (segment (start 126.34 96.1) (end 127 96.76) (width 0.25) (layer B.Cu) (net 16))
 (segment (start 109.21 96.1) (end 126.34 96.1) (width 0.25) (layer B.Cu) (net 16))
 (segment (start 107.96 97.35) (end 109.21 96.1) (width 0.25) (layer B.Cu) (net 16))
 (segment (start 169.873 94.81) (end 149.99 94.81) (width 0.25) (layer B.Cu) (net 12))
 (via (at 130.2 96.75) (size 0.6) (drill 0.4) (layers F.Cu B.Cu) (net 12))
 (segment (start 130.2 96.75) (end 130.2 95.35) (width 0.25) (layer F.Cu) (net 12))
 (segment (start 144.58 96.75) (end 130.2 96.75) (width 0.25) (layer B.Cu) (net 12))
 (segment (start 145.26 96.07) (end 144.58 96.75) (width 0.25) (layer B.Cu) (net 12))
 (segment (start 148.73 96.07) (end 145.26 96.07) (width 0.25) (layer B.Cu) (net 12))
 (segment (start 149.99 94.81) (end 148.73 96.07) (width 0.25) (layer B.Cu) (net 12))
 (segment (start 170.127 97.35) (end 150.03 97.35) (width 0.25) (layer B.Cu) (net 13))
 (via (at 129.4 97.57) (size 0.6) (drill 0.4) (layers F.Cu B.Cu) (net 13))
 (segment (start 129.4 97.57) (end 129.4 95.35) (width 0.25) (layer F.Cu) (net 13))
 (segment (start 130.45 98.62) (end 129.4 97.57) (width 0.25) (layer B.Cu) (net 13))
 (segment (start 148.76 98.62) (end 130.45 98.62) (width 0.25) (layer B.Cu) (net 13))
 (segment (start 150.03 97.35) (end 148.76 98.62) (width 0.25) (layer B.Cu) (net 13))
 (segment (start 169.873 84.65) (end 150.07 84.65) (width 0.25) (layer B.Cu) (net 5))
 (via (at 126.2 83.2) (size 0.6) (drill 0.4) (layers F.Cu B.Cu) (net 5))
 (segment (start 126.2 83.2) (end 126.2 86.65) (width 0.25) (layer F.Cu) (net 5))
 (segment (start 145.06 83.2) (end 126.2 83.2) (width 0.25) (layer B.Cu) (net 5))
 (segment (start 145.25 83.39) (end 145.06 83.2) (width 0.25) (layer B.Cu) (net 5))
 (segment (start 148.81 83.39) (end 145.25 83.39) (width 0.25) (layer B.Cu) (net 5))
 (segment (start 150.07 84.65) (end 148.81 83.39) (width 0.25) (layer B.Cu) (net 5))
 (segment (start 87.873 94.81) (end 107.96 94.81) (width 0.25) (layer B.Cu) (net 10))
 (via (at 122.76 91.4) (size 0.6) (drill 0.4) (layers F.Cu B.Cu) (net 10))
 (segment (start 122.76 91.4) (end 124.65 91.4) (width 0.25) (layer F.Cu) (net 10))
 (segment (start 120.62 93.54) (end 122.76 91.4) (width 0.25) (layer B.Cu) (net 10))
 (segment (start 109.23 93.54) (end 120.62 93.54) (width 0.25) (layer B.Cu) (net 10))
 (segment (start 107.96 94.81) (end 109.23 93.54) (width 0.25) (layer B.Cu) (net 10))
 (segment (start 87.873 89.73) (end 108.35 89.73) (width 0.25) (layer B.Cu) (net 8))
 (segment (start 114.2 89.8) (end 122.76 89.8) (width 0.25) (layer B.Cu) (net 8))
 (segment (start 112.87 88.47) (end 114.2 89.8) (width 0.25) (layer B.Cu) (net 8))
 (segment (start 109.61 88.47) (end 112.87 88.47) (width 0.25) (layer B.Cu) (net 8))
 (segment (start 108.35 89.73) (end 109.61 88.47) (width 0.25) (layer B.Cu) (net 8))
 (segment (start 124.65 89.8) (end 122.76 89.8) (width 0.25) (layer F.Cu) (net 8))
 (segment (start 122.76 89.8) (end 122.76 89.81) (width 0.25) (layer B.Cu) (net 8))
 (via (at 122.76 89.8) (size 0.6) (drill 0.4) (layers F.Cu B.Cu) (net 8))
 (segment (start 88.127 92.27) (end 107.47 92.27) (width 0.25) (layer B.Cu) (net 9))
 (segment (start 121.6 90.6) (end 124.65 90.6) (width 0.25) (layer F.Cu) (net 9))
 (via (at 121.6 90.6) (size 0.6) (drill 0.4) (layers F.Cu B.Cu) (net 9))
 (segment (start 121.17 91.03) (end 121.6 90.6) (width 0.25) (layer B.Cu) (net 9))
 (segment (start 108.71 91.03) (end 121.17 91.03) (width 0.25) (layer B.Cu) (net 9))
 (segment (start 107.47 92.27) (end 108.71 91.03) (width 0.25) (layer B.Cu) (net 9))
 (segment (start 170.127 87.19) (end 150.01 87.19) (width 0.25) (layer B.Cu) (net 4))
 (via (at 127 84.35) (size 0.6) (drill 0.4) (layers F.Cu B.Cu) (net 4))
 (segment (start 127 84.35) (end 127 86.65) (width 0.25) (layer F.Cu) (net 4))
 (segment (start 143.69 84.35) (end 127 84.35) (width 0.25) (layer B.Cu) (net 4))
 (segment (start 145.26 85.92) (end 143.69 84.35) (width 0.25) (layer B.Cu) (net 4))
 (segment (start 148.74 85.92) (end 145.26 85.92) (width 0.25) (layer B.Cu) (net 4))
 (segment (start 150.01 87.19) (end 148.74 85.92) (width 0.25) (layer B.Cu) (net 4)))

